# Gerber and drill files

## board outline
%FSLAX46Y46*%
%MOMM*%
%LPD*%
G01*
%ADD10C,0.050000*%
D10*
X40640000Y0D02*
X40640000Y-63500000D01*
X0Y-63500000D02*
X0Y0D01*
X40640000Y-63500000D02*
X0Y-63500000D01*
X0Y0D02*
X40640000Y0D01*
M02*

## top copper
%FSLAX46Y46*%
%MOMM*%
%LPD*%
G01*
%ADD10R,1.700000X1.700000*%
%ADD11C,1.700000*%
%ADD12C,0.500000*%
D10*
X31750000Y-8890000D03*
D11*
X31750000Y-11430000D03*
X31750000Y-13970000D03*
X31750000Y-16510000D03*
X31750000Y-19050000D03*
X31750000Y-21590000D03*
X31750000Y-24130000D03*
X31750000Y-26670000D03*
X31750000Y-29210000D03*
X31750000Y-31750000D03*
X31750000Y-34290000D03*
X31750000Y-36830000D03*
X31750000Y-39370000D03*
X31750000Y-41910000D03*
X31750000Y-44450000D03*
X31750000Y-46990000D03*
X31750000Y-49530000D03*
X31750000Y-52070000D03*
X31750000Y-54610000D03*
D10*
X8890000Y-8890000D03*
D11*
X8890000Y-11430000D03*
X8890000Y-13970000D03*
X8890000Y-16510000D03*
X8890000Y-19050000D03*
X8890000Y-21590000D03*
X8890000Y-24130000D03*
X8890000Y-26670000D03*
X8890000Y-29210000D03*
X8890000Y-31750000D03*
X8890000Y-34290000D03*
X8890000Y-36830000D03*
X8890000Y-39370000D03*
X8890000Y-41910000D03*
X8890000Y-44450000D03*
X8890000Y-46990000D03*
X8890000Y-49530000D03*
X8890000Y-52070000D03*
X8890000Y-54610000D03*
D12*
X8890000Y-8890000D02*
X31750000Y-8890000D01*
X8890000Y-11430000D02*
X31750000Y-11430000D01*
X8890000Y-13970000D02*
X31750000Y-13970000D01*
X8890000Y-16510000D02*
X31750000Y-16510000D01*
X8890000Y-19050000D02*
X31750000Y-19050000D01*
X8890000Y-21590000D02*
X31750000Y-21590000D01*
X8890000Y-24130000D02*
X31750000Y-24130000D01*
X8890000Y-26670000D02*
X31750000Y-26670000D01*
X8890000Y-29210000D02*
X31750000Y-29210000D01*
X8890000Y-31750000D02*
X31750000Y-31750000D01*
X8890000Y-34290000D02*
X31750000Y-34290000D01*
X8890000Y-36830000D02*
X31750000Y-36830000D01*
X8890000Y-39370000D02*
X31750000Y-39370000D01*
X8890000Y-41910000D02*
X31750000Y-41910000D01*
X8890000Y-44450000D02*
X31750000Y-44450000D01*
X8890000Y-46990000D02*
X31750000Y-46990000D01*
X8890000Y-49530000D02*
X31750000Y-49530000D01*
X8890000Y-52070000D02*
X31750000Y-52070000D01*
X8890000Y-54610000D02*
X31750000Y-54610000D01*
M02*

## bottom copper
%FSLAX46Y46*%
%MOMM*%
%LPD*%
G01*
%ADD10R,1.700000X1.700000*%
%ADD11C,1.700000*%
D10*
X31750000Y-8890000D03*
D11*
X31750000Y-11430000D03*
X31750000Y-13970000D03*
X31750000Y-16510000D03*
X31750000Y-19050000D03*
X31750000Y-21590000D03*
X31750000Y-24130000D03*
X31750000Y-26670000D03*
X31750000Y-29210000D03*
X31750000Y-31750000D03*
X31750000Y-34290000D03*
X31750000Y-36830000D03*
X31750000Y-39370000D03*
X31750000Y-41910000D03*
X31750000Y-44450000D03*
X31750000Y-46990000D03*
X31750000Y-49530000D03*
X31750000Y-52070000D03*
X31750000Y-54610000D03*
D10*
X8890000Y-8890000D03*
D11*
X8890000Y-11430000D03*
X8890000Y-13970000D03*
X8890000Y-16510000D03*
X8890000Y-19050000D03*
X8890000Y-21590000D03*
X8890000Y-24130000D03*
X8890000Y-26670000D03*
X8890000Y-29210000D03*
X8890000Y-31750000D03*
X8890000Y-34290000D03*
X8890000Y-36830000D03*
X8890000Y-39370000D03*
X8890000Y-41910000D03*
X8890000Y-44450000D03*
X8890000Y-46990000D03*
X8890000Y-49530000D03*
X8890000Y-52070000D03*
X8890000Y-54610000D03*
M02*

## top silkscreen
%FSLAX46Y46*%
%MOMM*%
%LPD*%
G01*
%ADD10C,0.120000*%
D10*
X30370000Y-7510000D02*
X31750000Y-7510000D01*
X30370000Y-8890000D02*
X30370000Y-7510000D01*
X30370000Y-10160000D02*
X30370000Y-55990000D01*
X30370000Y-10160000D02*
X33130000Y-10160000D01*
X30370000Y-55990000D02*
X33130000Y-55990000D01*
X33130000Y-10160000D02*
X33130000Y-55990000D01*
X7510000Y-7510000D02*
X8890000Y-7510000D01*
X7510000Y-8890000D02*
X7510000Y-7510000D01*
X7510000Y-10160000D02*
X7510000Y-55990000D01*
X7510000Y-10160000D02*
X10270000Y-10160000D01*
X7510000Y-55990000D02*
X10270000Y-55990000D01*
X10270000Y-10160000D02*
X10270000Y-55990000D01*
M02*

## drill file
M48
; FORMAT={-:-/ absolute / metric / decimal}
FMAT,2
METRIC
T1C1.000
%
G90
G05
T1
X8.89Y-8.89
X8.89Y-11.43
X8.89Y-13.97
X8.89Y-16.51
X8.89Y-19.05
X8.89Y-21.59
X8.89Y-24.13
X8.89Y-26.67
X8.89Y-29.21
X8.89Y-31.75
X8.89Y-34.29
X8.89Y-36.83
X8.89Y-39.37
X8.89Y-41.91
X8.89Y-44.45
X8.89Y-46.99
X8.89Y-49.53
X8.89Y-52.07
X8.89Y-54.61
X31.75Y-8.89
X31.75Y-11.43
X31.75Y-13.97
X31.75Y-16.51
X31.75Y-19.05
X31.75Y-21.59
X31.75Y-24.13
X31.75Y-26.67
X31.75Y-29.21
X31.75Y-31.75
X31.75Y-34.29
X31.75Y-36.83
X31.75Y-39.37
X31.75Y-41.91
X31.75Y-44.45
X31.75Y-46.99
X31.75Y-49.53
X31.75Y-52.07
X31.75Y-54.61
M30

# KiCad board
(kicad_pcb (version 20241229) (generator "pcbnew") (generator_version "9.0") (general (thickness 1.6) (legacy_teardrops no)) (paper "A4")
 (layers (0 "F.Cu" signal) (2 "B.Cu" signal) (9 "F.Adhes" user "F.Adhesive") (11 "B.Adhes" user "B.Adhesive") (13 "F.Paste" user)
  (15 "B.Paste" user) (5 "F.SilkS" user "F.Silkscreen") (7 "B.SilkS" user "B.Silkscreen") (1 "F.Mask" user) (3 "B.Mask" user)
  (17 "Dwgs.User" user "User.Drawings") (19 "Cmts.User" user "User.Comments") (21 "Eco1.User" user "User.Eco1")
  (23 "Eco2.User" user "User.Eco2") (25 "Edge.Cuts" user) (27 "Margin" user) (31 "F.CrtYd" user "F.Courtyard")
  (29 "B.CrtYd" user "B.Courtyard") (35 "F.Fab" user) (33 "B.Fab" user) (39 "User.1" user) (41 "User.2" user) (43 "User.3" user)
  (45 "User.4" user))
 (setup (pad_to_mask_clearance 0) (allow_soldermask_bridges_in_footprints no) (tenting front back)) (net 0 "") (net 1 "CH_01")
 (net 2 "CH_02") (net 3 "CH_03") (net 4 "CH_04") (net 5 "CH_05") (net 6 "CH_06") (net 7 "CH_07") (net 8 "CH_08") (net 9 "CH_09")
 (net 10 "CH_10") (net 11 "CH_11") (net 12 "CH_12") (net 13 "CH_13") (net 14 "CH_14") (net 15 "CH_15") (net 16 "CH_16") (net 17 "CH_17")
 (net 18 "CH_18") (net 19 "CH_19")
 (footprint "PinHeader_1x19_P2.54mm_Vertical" (layer "F.Cu") (at 31.75 8.89)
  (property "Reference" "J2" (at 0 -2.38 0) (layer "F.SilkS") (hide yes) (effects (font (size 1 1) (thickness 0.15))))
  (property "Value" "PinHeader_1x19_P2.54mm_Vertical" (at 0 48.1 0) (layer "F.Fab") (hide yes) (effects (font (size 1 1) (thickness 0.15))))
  (fp_line (start -1.38 -1.38) (end 0 -1.38) (stroke (width 0.12) (type solid)) (layer "F.SilkS"))
  (fp_line (start -1.38 0) (end -1.38 -1.38) (stroke (width 0.12) (type solid)) (layer "F.SilkS"))
  (fp_line (start -1.38 1.27) (end -1.38 47.1) (stroke (width 0.12) (type solid)) (layer "F.SilkS"))
  (fp_line (start -1.38 1.27) (end 1.38 1.27) (stroke (width 0.12) (type solid)) (layer "F.SilkS"))
  (fp_line (start -1.38 47.1) (end 1.38 47.1) (stroke (width 0.12) (type solid)) (layer "F.SilkS"))
  (fp_line (start 1.38 1.27) (end 1.38 47.1) (stroke (width 0.12) (type solid)) (layer "F.SilkS"))
  (pad "1" thru_hole rect (at 0 0) (size 1.7 1.7) (drill 1) (layers "*.Cu" "*.Mask") (remove_unused_layers no) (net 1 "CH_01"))
  (pad "2" thru_hole circle (at 0 2.54) (size 1.7 1.7) (drill 1) (layers "*.Cu" "*.Mask") (remove_unused_layers no) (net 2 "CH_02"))
  (pad "3" thru_hole circle (at 0 5.08) (size 1.7 1.7) (drill 1) (layers "*.Cu" "*.Mask") (remove_unused_layers no) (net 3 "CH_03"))
  (pad "4" thru_hole circle (at 0 7.62) (size 1.7 1.7) (drill 1) (layers "*.Cu" "*.Mask") (remove_unused_layers no) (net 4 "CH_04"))
  (pad "5" thru_hole circle (at 0 10.16) (size 1.7 1.7) (drill 1) (layers "*.Cu" "*.Mask") (remove_unused_layers no) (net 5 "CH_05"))
  (pad "6" thru_hole circle (at 0 12.7) (size 1.7 1.7) (drill 1) (layers "*.Cu" "*.Mask") (remove_unused_layers no) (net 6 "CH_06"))
  (pad "7" thru_hole circle (at 0 15.24) (size 1.7 1.7) (drill 1) (layers "*.Cu" "*.Mask") (remove_unused_layers no) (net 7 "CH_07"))
  (pad "8" thru_hole circle (at 0 17.78) (size 1.7 1.7) (drill 1) (layers "*.Cu" "*.Mask") (remove_unused_layers no) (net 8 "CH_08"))
  (pad "9" thru_hole circle (at 0 20.32) (size 1.7 1.7) (drill 1) (layers "*.Cu" "*.Mask") (remove_unused_layers no) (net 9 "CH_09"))
  (pad "10" thru_hole circle (at 0 22.86) (size 1.7 1.7) (drill 1) (layers "*.Cu" "*.Mask") (remove_unused_layers no) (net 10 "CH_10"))
  (pad "11" thru_hole circle (at 0 25.4) (size 1.7 1.7) (drill 1) (layers "*.Cu" "*.Mask") (remove_unused_layers no) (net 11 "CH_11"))
  (pad "12" thru_hole circle (at 0 27.94) (size 1.7 1.7) (drill 1) (layers "*.Cu" "*.Mask") (remove_unused_layers no) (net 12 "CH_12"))
  (pad "13" thru_hole circle (at 0 30.48) (size 1.7 1.7) (drill 1) (layers "*.Cu" "*.Mask") (remove_unused_layers no) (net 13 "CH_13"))
  (pad "14" thru_hole circle (at 0 33.02) (size 1.7 1.7) (drill 1) (layers "*.Cu" "*.Mask") (remove_unused_layers no) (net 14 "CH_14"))
  (pad "15" thru_hole circle (at 0 35.56) (size 1.7 1.7) (drill 1) (layers "*.Cu" "*.Mask") (remove_unused_layers no) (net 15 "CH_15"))
  (pad "16" thru_hole circle (at 0 38.1) (size 1.7 1.7) (drill 1) (layers "*.Cu" "*.Mask") (remove_unused_layers no) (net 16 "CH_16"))
  (pad "17" thru_hole circle (at 0 40.64) (size 1.7 1.7) (drill 1) (layers "*.Cu" "*.Mask") (remove_unused_layers no) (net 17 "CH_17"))
  (pad "18" thru_hole circle (at 0 43.18) (size 1.7 1.7) (drill 1) (layers "*.Cu" "*.Mask") (remove_unused_layers no) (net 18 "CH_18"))
  (pad "19" thru_hole circle (at 0 45.72) (size 1.7 1.7) (drill 1) (layers "*.Cu" "*.Mask") (remove_unused_layers no) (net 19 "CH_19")))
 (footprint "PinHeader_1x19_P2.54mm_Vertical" (layer "F.Cu") (at 8.89 8.89)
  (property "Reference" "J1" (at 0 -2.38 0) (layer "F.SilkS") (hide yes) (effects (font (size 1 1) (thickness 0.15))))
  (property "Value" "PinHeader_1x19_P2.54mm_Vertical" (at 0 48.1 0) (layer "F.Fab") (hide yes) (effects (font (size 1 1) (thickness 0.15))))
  (fp_line (start -1.38 -1.38) (end 0 -1.38) (stroke (width 0.12) (type solid)) (layer "F.SilkS"))
  (fp_line (start -1.38 0) (end -1.38 -1.38) (stroke (width 0.12) (type solid)) (layer "F.SilkS"))
  (fp_line (start -1.38 1.27) (end -1.38 47.1) (stroke (width 0.12) (type solid)) (layer "F.SilkS"))
  (fp_line (start -1.38 1.27) (end 1.38 1.27) (stroke (width 0.12) (type solid)) (layer "F.SilkS"))
  (fp_line (start -1.38 47.1) (end 1.38 47.1) (stroke (width 0.12) (type solid)) (layer "F.SilkS"))
  (fp_line (start 1.38 1.27) (end 1.38 47.1) (stroke (width 0.12) (type solid)) (layer "F.SilkS"))
  (pad "1" thru_hole rect (at 0 0) (size 1.7 1.7) (drill 1) (layers "*.Cu" "*.Mask") (remove_unused_layers no) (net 1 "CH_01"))
  (pad "2" thru_hole circle (at 0 2.54) (size 1.7 1.7) (drill 1) (layers "*.Cu" "*.Mask") (remove_unused_layers no) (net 2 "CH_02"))
  (pad "3" thru_hole circle (at 0 5.08) (size 1.7 1.7) (drill 1) (layers "*.Cu" "*.Mask") (remove_unused_layers no) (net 3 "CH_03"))
  (pad "4" thru_hole circle (at 0 7.62) (size 1.7 1.7) (drill 1) (layers "*.Cu" "*.Mask") (remove_unused_layers no) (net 4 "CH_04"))
  (pad "5" thru_hole circle (at 0 10.16) (size 1.7 1.7) (drill 1) (layers "*.Cu" "*.Mask") (remove_unused_layers no) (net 5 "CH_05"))
  (pad "6" thru_hole circle (at 0 12.7) (size 1.7 1.7) (drill 1) (layers "*.Cu" "*.Mask") (remove_unused_layers no) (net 6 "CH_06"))
  (pad "7" thru_hole circle (at 0 15.24) (size 1.7 1.7) (drill 1) (layers "*.Cu" "*.Mask") (remove_unused_layers no) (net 7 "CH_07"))
  (pad "8" thru_hole circle (at 0 17.78) (size 1.7 1.7) (drill 1) (layers "*.Cu" "*.Mask") (remove_unused_layers no) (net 8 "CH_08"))
  (pad "9" thru_hole circle (at 0 20.32) (size 1.7 1.7) (drill 1) (layers "*.Cu" "*.Mask") (remove_unused_layers no) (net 9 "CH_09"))
  (pad "10" thru_hole circle (at 0 22.86) (size 1.7 1.7) (drill 1) (layers "*.Cu" "*.Mask") (remove_unused_layers no) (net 10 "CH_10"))
  (pad "11" thru_hole circle (at 0 25.4) (size 1.7 1.7) (drill 1) (layers "*.Cu" "*.Mask") (remove_unused_layers no) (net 11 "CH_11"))
  (pad "12" thru_hole circle (at 0 27.94) (size 1.7 1.7) (drill 1) (layers "*.Cu" "*.Mask") (remove_unused_layers no) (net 12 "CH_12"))
  (pad "13" thru_hole circle (at 0 30.48) (size 1.7 1.7) (drill 1) (layers "*.Cu" "*.Mask") (remove_unused_layers no) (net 13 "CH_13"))
  (pad "14" thru_hole circle (at 0 33.02) (size 1.7 1.7) (drill 1) (layers "*.Cu" "*.Mask") (remove_unused_layers no) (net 14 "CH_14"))
  (pad "15" thru_hole circle (at 0 35.56) (size 1.7 1.7) (drill 1) (layers "*.Cu" "*.Mask") (remove_unused_layers no) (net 15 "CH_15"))
  (pad "16" thru_hole circle (at 0 38.1) (size 1.7 1.7) (drill 1) (layers "*.Cu" "*.Mask") (remove_unused_layers no) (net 16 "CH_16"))
  (pad "17" thru_hole circle (at 0 40.64) (size 1.7 1.7) (drill 1) (layers "*.Cu" "*.Mask") (remove_unused_layers no) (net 17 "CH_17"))
  (pad "18" thru_hole circle (at 0 43.18) (size 1.7 1.7) (drill 1) (layers "*.Cu" "*.Mask") (remove_unused_layers no) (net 18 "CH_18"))
  (pad "19" thru_hole circle (at 0 45.72) (size 1.7 1.7) (drill 1) (layers "*.Cu" "*.Mask") (remove_unused_layers no) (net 19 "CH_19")))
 (gr_line (start 40.64 0) (end 40.64 63.5) (stroke (width 0.05) (type default)) (layer "Edge.Cuts"))
 (gr_line (start 0 63.5) (end 0 0) (stroke (width 0.05) (type default)) (layer "Edge.Cuts"))
 (gr_line (start 40.64 63.5) (end 0 63.5) (stroke (width 0.05) (type default)) (layer "Edge.Cuts"))
 (gr_line (start 0 0) (end 40.64 0) (stroke (width 0.05) (type default)) (layer "Edge.Cuts"))
 (segment (start 8.89 8.89) (end 31.75 8.89) (width 0.5) (layer "F.Cu") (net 1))
 (segment (start 8.89 11.43) (end 31.75 11.43) (width 0.5) (layer "F.Cu") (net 2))
 (segment (start 8.89 13.97) (end 31.75 13.97) (width 0.5) (layer "F.Cu") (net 3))
 (segment (start 8.89 16.51) (end 31.75 16.51) (width 0.5) (layer "F.Cu") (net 4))
 (segment (start 8.89 19.05) (end 31.75 19.05) (width 0.5) (layer "F.Cu") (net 5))
 (segment (start 8.89 21.59) (end 31.75 21.59) (width 0.5) (layer "F.Cu") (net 6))
 (segment (start 8.89 24.13) (end 31.75 24.13) (width 0.5) (layer "F.Cu") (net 7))
 (segment (start 8.89 26.67) (end 31.75 26.67) (width 0.5) (layer "F.Cu") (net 8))
 (segment (start 8.89 29.21) (end 31.75 29.21) (width 0.5) (layer "F.Cu") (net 9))
 (segment (start 8.89 31.75) (end 31.75 31.75) (width 0.5) (layer "F.Cu") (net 10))
 (segment (start 8.89 34.29) (end 31.75 34.29) (width 0.5) (layer "F.Cu") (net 11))
 (segment (start 8.89 36.83) (end 31.75 36.83) (width 0.5) (layer "F.Cu") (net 12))
 (segment (start 8.89 39.37) (end 31.75 39.37) (width 0.5) (layer "F.Cu") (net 13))
 (segment (start 8.89 41.91) (end 31.75 41.91) (width 0.5) (layer "F.Cu") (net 14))
 (segment (start 8.89 44.45) (end 31.75 44.45) (width 0.5) (layer "F.Cu") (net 15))
 (segment (start 8.89 46.99) (end 31.75 46.99) (width 0.5) (layer "F.Cu") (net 16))
 (segment (start 8.89 49.53) (end 31.75 49.53) (width 0.5) (layer "F.Cu") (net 17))
 (segment (start 8.89 52.07) (end 31.75 52.07) (width 0.5) (layer "F.Cu") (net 18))
 (segment (start 8.89 54.61) (end 31.75 54.61) (width 0.5) (layer "F.Cu") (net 19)))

